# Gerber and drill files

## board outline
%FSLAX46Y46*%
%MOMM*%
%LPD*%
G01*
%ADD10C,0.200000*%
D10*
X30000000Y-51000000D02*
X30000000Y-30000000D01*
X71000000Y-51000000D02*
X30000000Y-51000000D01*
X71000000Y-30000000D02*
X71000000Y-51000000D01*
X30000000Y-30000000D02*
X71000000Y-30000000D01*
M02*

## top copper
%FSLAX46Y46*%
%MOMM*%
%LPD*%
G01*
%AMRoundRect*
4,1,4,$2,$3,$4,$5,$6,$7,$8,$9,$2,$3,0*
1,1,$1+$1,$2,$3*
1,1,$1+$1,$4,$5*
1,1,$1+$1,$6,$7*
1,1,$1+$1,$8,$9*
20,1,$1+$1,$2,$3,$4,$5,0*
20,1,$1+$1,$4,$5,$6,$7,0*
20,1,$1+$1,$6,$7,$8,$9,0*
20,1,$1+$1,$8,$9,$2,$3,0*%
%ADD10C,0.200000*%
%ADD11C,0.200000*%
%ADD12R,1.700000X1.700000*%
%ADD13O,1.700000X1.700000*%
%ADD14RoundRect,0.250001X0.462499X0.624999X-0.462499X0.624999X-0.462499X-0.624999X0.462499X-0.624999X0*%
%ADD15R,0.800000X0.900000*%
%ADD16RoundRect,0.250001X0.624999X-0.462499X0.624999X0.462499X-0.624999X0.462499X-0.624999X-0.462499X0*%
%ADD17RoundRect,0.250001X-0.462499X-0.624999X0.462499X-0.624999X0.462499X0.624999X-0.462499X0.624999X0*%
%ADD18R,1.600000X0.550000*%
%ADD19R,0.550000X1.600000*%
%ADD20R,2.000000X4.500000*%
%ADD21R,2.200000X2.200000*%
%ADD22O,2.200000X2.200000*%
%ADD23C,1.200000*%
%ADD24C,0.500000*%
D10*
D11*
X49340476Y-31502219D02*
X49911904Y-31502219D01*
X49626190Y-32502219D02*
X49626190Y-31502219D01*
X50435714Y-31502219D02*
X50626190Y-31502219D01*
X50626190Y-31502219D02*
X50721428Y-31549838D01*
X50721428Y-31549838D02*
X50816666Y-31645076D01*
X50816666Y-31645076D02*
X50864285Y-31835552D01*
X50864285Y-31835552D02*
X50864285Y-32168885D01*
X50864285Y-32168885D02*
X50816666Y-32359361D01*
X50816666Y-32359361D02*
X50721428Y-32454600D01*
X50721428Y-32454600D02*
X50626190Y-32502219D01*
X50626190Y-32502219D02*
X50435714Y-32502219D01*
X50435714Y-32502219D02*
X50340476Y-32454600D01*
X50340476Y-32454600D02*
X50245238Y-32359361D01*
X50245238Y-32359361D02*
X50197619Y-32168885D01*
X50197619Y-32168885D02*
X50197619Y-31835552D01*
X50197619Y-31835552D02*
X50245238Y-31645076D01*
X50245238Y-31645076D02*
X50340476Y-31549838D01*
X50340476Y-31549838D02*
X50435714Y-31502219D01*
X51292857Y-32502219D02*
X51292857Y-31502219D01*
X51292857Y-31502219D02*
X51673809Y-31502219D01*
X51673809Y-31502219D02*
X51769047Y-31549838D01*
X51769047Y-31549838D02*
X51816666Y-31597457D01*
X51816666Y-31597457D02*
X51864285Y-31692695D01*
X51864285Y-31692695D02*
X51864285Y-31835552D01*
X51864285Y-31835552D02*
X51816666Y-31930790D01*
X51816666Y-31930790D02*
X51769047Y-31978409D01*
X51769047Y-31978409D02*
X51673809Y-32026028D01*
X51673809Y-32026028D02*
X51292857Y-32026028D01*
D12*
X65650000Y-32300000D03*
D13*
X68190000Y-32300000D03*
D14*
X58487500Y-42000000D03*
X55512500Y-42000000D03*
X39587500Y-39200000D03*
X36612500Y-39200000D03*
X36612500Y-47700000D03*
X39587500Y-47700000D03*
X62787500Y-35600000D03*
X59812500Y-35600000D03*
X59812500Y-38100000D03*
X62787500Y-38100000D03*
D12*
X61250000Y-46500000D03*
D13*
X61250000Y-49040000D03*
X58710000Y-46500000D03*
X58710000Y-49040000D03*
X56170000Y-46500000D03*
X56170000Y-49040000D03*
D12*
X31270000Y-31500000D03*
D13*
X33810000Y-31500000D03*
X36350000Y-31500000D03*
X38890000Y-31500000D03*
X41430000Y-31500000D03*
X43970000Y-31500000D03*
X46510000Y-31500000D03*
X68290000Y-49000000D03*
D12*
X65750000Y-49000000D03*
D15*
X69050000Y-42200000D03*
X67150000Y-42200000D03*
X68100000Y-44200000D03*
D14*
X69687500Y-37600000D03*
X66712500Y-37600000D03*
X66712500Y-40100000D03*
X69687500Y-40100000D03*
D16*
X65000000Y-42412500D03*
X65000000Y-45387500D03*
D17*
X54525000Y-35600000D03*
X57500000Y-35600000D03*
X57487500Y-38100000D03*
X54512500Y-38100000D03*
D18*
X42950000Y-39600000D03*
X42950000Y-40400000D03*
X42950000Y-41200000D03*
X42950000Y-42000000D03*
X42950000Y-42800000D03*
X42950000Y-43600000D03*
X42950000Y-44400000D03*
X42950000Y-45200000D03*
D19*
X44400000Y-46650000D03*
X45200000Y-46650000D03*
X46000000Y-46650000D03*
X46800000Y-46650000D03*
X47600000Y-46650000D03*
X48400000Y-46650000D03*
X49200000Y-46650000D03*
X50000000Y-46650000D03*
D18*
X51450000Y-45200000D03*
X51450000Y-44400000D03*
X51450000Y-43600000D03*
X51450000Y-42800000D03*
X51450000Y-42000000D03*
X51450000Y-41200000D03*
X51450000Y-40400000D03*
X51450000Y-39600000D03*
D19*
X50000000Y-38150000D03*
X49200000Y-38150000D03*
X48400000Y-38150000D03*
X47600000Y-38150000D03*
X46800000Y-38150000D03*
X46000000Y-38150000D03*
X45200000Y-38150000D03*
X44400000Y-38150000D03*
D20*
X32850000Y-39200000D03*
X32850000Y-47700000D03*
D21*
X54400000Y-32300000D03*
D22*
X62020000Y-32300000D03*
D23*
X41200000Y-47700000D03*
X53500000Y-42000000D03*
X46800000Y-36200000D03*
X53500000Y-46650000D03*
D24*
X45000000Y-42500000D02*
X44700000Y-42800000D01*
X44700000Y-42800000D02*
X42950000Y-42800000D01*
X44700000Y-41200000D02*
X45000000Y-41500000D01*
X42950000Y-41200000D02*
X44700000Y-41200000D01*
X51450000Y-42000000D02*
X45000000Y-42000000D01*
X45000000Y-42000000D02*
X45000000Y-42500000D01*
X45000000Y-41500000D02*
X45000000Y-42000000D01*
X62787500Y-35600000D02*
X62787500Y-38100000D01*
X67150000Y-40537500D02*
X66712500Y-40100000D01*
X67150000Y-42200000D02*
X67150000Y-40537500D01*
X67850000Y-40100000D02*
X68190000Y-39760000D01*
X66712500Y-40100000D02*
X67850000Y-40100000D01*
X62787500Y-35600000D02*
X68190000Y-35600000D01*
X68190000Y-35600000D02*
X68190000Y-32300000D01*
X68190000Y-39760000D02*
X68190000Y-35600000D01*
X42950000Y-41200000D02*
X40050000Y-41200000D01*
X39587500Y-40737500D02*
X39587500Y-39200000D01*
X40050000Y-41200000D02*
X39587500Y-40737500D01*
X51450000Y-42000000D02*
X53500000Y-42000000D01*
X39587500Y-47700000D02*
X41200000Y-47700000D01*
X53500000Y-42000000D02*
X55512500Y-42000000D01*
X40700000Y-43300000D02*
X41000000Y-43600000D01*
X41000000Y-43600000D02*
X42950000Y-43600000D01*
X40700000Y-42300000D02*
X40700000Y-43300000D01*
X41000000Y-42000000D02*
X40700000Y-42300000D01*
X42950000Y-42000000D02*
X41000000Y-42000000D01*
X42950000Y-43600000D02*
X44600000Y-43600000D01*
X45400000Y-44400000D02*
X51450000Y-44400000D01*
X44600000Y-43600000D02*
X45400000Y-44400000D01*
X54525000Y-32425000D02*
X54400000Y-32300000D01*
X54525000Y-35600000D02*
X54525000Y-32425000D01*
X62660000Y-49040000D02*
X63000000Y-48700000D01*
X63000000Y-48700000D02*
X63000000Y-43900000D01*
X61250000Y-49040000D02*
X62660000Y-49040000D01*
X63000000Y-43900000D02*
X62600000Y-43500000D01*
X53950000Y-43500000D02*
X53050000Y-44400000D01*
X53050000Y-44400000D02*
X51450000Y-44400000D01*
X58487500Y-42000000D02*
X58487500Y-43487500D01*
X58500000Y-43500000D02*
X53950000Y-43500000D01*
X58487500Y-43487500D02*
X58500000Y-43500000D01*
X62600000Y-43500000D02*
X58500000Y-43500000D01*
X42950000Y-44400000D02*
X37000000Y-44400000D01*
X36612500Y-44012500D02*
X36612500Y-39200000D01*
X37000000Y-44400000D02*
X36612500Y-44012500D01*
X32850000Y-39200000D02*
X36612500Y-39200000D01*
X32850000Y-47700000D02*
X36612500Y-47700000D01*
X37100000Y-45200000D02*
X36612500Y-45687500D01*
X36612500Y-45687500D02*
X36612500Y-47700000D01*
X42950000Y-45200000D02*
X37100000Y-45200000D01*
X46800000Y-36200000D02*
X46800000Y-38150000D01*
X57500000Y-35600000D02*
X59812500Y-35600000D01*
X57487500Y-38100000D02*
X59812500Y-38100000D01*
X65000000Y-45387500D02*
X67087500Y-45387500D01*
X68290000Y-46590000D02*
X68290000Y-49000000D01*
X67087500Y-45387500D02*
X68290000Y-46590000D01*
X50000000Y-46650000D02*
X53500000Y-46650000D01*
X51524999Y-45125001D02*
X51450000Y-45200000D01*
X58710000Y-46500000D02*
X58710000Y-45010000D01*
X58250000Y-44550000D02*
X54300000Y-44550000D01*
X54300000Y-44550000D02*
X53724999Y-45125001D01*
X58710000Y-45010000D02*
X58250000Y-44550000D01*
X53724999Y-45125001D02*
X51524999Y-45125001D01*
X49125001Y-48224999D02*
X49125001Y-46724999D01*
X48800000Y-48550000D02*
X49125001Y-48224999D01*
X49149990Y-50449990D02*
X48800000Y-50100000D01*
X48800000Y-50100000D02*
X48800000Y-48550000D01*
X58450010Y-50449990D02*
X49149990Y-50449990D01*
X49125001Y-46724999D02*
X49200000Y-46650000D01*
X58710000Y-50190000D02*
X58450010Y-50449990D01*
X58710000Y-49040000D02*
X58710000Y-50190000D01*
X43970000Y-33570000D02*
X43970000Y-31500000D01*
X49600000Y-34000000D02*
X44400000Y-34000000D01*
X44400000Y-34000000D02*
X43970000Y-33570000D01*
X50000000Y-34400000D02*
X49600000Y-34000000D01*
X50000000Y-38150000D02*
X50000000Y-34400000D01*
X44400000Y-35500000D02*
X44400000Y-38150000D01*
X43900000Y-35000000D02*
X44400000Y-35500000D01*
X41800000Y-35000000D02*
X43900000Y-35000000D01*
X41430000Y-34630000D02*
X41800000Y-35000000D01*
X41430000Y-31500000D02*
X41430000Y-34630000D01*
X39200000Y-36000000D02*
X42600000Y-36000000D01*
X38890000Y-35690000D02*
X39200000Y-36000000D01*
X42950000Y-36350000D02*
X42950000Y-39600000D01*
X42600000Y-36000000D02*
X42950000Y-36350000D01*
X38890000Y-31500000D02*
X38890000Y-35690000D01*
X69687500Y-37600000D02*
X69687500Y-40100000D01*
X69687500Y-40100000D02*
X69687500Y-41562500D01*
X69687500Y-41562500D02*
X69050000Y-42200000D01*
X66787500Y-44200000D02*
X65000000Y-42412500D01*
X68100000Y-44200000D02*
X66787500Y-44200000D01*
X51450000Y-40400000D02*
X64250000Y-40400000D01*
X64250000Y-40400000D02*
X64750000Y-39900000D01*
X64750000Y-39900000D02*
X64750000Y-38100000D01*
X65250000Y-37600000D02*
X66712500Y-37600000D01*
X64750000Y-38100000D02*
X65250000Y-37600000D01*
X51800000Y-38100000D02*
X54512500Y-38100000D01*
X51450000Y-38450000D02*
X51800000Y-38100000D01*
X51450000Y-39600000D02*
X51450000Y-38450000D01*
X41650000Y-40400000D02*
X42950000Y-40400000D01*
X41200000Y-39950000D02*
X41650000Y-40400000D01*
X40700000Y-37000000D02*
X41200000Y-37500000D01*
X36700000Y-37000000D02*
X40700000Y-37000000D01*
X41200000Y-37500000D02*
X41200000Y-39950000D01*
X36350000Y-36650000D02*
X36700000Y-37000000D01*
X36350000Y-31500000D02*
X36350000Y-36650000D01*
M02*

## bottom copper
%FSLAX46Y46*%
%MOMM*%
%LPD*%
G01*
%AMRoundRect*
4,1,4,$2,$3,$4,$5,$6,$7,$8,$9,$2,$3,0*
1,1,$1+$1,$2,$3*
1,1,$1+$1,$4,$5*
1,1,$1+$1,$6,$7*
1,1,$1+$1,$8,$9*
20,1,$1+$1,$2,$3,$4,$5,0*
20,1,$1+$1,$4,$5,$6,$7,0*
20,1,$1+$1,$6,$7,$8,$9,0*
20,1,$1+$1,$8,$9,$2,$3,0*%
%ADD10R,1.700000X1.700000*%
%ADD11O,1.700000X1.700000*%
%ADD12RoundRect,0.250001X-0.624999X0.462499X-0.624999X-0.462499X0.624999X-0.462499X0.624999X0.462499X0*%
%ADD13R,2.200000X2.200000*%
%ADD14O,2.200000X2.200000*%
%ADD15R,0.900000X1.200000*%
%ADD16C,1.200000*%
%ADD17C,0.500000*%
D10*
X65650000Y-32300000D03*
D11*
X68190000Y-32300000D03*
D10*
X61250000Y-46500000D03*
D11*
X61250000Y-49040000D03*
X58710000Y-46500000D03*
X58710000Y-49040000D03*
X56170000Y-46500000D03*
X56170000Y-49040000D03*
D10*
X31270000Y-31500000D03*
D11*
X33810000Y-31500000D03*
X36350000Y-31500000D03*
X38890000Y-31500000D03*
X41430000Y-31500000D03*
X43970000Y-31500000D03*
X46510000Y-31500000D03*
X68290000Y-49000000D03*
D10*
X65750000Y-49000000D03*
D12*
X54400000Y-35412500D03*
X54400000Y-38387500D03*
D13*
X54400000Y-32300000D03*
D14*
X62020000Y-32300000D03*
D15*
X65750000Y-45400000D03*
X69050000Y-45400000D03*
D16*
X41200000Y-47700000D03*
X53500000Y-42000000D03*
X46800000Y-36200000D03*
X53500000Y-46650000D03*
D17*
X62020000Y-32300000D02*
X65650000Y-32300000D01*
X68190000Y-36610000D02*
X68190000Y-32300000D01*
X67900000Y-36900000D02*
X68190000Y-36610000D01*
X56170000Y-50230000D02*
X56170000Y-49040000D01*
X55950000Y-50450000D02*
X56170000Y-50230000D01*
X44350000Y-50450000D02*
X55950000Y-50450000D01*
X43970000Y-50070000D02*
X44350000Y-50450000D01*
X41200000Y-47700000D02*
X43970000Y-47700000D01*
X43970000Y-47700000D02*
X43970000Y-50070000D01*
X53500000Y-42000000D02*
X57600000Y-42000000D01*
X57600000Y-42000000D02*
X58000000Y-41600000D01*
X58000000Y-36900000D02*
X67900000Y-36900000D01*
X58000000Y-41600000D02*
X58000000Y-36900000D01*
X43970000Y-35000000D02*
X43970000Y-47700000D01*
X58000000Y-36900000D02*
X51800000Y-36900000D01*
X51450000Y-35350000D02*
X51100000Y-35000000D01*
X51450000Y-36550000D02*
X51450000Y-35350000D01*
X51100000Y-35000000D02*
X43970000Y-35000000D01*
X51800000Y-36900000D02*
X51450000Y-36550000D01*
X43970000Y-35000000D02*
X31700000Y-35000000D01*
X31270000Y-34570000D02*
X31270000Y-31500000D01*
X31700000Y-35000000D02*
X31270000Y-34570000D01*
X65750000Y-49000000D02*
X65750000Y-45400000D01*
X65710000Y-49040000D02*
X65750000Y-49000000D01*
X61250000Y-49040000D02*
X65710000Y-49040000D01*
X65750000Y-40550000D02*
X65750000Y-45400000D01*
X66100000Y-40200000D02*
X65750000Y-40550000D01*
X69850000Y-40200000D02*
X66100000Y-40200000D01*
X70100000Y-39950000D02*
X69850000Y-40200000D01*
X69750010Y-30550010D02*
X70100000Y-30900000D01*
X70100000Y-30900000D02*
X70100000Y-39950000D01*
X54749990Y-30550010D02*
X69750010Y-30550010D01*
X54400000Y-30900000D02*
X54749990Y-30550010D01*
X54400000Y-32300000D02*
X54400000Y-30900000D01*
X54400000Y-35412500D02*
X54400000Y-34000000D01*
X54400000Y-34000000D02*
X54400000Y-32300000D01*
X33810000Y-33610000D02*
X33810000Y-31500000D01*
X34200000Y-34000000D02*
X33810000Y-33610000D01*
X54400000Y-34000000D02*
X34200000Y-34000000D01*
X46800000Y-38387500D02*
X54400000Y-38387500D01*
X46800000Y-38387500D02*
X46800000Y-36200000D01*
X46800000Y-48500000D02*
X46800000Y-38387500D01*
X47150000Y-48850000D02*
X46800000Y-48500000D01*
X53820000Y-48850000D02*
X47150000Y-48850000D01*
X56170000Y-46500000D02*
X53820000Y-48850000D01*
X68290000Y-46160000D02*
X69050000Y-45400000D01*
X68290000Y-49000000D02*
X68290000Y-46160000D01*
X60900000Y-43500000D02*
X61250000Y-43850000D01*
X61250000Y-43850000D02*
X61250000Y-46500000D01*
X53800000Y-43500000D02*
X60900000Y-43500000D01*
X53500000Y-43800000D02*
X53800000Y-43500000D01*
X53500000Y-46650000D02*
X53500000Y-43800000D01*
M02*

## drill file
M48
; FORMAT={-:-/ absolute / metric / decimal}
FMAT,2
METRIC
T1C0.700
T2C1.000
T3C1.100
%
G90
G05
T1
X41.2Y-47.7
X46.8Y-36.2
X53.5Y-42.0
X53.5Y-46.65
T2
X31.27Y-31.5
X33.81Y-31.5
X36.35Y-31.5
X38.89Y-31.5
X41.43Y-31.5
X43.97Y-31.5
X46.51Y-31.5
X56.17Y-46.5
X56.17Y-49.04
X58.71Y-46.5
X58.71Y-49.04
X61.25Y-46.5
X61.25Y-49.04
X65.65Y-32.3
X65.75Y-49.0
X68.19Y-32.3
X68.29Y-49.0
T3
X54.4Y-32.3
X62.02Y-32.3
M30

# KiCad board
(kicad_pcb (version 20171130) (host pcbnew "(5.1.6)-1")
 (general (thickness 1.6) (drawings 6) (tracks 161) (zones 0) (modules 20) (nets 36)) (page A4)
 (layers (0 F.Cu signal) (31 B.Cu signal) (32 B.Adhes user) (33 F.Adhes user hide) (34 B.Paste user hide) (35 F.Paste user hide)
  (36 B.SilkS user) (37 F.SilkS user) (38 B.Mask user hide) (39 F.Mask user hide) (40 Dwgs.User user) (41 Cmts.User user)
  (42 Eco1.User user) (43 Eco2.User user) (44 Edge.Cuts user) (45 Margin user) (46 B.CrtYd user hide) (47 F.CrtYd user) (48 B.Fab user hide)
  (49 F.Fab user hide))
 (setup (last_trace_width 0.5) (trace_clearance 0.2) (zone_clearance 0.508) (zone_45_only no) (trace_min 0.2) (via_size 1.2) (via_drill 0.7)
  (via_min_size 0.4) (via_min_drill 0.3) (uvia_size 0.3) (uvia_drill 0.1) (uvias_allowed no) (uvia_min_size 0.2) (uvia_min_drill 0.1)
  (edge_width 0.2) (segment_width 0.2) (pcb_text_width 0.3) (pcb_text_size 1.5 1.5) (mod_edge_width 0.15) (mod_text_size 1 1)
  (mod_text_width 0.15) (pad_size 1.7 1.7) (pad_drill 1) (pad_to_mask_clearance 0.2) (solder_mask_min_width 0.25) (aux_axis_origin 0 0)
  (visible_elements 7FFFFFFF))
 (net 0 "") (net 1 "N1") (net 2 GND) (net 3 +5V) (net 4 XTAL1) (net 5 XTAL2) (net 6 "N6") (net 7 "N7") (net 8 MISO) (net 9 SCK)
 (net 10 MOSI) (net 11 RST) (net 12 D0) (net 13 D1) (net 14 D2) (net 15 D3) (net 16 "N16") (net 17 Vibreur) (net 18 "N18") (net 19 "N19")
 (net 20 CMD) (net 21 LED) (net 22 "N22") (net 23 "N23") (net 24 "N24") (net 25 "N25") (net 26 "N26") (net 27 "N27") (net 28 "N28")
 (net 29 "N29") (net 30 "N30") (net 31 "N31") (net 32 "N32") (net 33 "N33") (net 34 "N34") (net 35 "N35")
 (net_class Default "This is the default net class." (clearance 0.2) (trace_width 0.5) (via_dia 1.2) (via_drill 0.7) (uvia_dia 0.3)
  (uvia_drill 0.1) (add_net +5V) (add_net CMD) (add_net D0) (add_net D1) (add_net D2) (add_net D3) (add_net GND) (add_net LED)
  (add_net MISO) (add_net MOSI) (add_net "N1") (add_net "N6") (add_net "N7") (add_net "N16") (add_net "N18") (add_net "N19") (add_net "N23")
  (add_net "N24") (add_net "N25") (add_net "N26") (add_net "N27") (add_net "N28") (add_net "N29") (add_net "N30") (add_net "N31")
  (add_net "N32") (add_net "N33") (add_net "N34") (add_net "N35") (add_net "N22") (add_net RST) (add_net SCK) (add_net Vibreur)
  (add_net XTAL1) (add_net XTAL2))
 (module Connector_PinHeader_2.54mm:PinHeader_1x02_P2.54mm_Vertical (layer F.Cu) (at 65.65 32.3 90)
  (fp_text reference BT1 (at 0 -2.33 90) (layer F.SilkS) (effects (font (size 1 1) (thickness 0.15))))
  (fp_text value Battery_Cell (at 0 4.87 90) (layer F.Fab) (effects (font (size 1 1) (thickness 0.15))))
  (pad 1 thru_hole rect (at 0 0 90) (size 1.7 1.7) (drill 1) (layers *.Cu *.Mask) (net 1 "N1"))
  (pad 2 thru_hole oval (at 0 2.54 90) (size 1.7 1.7) (drill 1) (layers *.Cu *.Mask) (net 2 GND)))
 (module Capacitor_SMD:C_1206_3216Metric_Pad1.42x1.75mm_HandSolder (layer F.Cu) (at 57 42 180)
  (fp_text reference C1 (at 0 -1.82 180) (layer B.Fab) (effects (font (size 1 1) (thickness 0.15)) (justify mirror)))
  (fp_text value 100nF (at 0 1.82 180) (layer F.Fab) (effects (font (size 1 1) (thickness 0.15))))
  (pad 1 smd roundrect (at -1.4875 0 180) (size 1.425 1.75) (layers F.Cu F.Paste F.Mask) (roundrect_rratio 0.175439) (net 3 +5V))
  (pad 2 smd roundrect (at 1.4875 0 180) (size 1.425 1.75) (layers F.Cu F.Paste F.Mask) (roundrect_rratio 0.175439) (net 2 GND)))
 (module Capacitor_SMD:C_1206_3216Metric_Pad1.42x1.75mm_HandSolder (layer F.Cu) (at 38.1 39.2 180)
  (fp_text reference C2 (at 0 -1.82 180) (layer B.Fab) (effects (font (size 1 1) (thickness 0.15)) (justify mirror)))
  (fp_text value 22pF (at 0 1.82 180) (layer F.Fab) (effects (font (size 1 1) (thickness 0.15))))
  (pad 1 smd roundrect (at -1.4875 0 180) (size 1.425 1.75) (layers F.Cu F.Paste F.Mask) (roundrect_rratio 0.175439) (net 2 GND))
  (pad 2 smd roundrect (at 1.4875 0 180) (size 1.425 1.75) (layers F.Cu F.Paste F.Mask) (roundrect_rratio 0.175439) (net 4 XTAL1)))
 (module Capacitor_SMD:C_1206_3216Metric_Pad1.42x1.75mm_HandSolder (layer F.Cu) (at 38.1 47.7 180)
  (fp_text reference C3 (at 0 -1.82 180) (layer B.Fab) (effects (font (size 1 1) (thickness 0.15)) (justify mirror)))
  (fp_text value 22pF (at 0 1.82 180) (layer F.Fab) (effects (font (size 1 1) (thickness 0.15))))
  (pad 2 smd roundrect (at 1.4875 0 180) (size 1.425 1.75) (layers F.Cu F.Paste F.Mask) (roundrect_rratio 0.175439) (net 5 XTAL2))
  (pad 1 smd roundrect (at -1.4875 0 180) (size 1.425 1.75) (layers F.Cu F.Paste F.Mask) (roundrect_rratio 0.175439) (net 2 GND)))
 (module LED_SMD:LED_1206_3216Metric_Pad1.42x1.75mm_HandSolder (layer F.Cu) (at 61.3 35.6 180)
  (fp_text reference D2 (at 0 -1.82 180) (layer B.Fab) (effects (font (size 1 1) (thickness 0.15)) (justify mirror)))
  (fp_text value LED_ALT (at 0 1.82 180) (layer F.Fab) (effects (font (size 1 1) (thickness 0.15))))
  (pad 1 smd roundrect (at -1.4875 0 180) (size 1.425 1.75) (layers F.Cu F.Paste F.Mask) (roundrect_rratio 0.175439) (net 2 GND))
  (pad 2 smd roundrect (at 1.4875 0 180) (size 1.425 1.75) (layers F.Cu F.Paste F.Mask) (roundrect_rratio 0.175439) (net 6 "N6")))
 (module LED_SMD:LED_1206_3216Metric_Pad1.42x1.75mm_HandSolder (layer F.Cu) (at 61.3 38.1 180)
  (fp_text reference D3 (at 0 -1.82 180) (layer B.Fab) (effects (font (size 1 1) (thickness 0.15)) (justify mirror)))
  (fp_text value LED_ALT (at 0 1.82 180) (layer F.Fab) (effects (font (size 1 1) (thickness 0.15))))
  (pad 2 smd roundrect (at 1.4875 0 180) (size 1.425 1.75) (layers F.Cu F.Paste F.Mask) (roundrect_rratio 0.175439) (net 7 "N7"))
  (pad 1 smd roundrect (at -1.4875 0 180) (size 1.425 1.75) (layers F.Cu F.Paste F.Mask) (roundrect_rratio 0.175439) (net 2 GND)))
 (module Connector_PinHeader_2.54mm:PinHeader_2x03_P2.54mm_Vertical (layer F.Cu) (at 61.25 46.5 270)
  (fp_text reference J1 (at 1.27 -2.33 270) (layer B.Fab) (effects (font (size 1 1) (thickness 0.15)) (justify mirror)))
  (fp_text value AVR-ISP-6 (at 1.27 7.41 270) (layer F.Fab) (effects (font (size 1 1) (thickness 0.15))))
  (pad 1 thru_hole rect (at 0 0 270) (size 1.7 1.7) (drill 1) (layers *.Cu *.Mask) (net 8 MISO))
  (pad 2 thru_hole oval (at 2.54 0 270) (size 1.7 1.7) (drill 1) (layers *.Cu *.Mask) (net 3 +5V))
  (pad 3 thru_hole oval (at 0 2.54 270) (size 1.7 1.7) (drill 1) (layers *.Cu *.Mask) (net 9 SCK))
  (pad 4 thru_hole oval (at 2.54 2.54 270) (size 1.7 1.7) (drill 1) (layers *.Cu *.Mask) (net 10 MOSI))
  (pad 5 thru_hole oval (at 0 5.08 270) (size 1.7 1.7) (drill 1) (layers *.Cu *.Mask) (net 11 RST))
  (pad 6 thru_hole oval (at 2.54 5.08 270) (size 1.7 1.7) (drill 1) (layers *.Cu *.Mask) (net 2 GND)))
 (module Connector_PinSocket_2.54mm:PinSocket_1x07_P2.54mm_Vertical (layer F.Cu) (at 31.27 31.5 90)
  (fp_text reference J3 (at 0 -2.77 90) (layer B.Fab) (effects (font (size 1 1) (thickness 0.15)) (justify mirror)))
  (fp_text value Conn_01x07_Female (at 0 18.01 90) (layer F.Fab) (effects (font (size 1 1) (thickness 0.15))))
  (pad 1 thru_hole rect (at 0 0 90) (size 1.7 1.7) (drill 1) (layers *.Cu *.Mask) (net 2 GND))
  (pad 2 thru_hole oval (at 0 2.54 90) (size 1.7 1.7) (drill 1) (layers *.Cu *.Mask) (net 3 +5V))
  (pad 3 thru_hole oval (at 0 5.08 90) (size 1.7 1.7) (drill 1) (layers *.Cu *.Mask) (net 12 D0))
  (pad 4 thru_hole oval (at 0 7.62 90) (size 1.7 1.7) (drill 1) (layers *.Cu *.Mask) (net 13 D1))
  (pad 5 thru_hole oval (at 0 10.16 90) (size 1.7 1.7) (drill 1) (layers *.Cu *.Mask) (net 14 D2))
  (pad 6 thru_hole oval (at 0 12.7 90) (size 1.7 1.7) (drill 1) (layers *.Cu *.Mask) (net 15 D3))
  (pad 7 thru_hole oval (at 0 15.24 90) (size 1.7 1.7) (drill 1) (layers *.Cu *.Mask) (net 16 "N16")))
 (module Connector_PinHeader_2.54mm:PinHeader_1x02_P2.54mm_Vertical (layer F.Cu) (at 65.75 49 90)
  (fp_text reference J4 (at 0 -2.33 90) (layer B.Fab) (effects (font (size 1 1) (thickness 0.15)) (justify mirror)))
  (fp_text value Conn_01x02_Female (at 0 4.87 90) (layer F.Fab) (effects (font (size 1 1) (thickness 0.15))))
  (pad 2 thru_hole oval (at 0 2.54 90) (size 1.7 1.7) (drill 1) (layers *.Cu *.Mask) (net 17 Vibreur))
  (pad 1 thru_hole rect (at 0 0 90) (size 1.7 1.7) (drill 1) (layers *.Cu *.Mask) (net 3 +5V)))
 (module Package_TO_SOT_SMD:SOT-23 (layer F.Cu) (at 68.1 43.2 270)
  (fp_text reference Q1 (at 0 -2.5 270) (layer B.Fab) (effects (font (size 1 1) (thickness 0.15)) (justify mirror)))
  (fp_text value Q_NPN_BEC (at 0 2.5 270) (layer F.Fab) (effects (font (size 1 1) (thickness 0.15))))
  (pad 1 smd rect (at -1 -0.95 270) (size 0.9 0.8) (layers F.Cu F.Paste F.Mask) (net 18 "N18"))
  (pad 2 smd rect (at -1 0.95 270) (size 0.9 0.8) (layers F.Cu F.Paste F.Mask) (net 2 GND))
  (pad 3 smd rect (at 1 0 270) (size 0.9 0.8) (layers F.Cu F.Paste F.Mask) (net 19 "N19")))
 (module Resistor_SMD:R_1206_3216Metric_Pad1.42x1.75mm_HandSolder (layer B.Cu) (at 54.4 36.9 270)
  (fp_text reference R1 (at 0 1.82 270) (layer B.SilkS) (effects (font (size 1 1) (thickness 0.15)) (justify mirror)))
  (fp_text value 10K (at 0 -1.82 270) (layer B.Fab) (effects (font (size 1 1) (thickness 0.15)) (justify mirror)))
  (pad 1 smd roundrect (at -1.4875 0 270) (size 1.425 1.75) (layers B.Cu B.Paste B.Mask) (roundrect_rratio 0.175439) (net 3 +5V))
  (pad 2 smd roundrect (at 1.4875 0 270) (size 1.425 1.75) (layers B.Cu B.Paste B.Mask) (roundrect_rratio 0.175439) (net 11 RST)))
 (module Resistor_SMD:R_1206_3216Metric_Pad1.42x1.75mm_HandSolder (layer F.Cu) (at 68.2 37.6 180)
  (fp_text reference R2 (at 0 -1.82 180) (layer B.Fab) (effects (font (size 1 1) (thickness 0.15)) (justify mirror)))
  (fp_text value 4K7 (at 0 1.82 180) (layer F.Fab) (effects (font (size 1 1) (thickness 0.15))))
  (pad 1 smd roundrect (at -1.4875 0 180) (size 1.425 1.75) (layers F.Cu F.Paste F.Mask) (roundrect_rratio 0.175439) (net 18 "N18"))
  (pad 2 smd roundrect (at 1.4875 0 180) (size 1.425 1.75) (layers F.Cu F.Paste F.Mask) (roundrect_rratio 0.175439) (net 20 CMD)))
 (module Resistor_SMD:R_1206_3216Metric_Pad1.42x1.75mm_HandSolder (layer F.Cu) (at 68.2 40.1 180)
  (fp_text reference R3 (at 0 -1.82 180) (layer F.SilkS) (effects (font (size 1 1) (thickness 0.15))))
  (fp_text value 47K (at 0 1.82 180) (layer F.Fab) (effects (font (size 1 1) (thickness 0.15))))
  (pad 2 smd roundrect (at 1.4875 0 180) (size 1.425 1.75) (layers F.Cu F.Paste F.Mask) (roundrect_rratio 0.175439) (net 2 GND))
  (pad 1 smd roundrect (at -1.4875 0 180) (size 1.425 1.75) (layers F.Cu F.Paste F.Mask) (roundrect_rratio 0.175439) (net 18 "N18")))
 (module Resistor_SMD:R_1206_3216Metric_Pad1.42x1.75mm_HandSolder (layer F.Cu) (at 65 43.9 90)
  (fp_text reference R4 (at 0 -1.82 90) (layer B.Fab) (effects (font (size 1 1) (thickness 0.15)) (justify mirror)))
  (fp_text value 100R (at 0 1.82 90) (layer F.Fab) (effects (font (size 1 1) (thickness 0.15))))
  (pad 2 smd roundrect (at 1.4875 0 90) (size 1.425 1.75) (layers F.Cu F.Paste F.Mask) (roundrect_rratio 0.175439) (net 19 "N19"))
  (pad 1 smd roundrect (at -1.4875 0 90) (size 1.425 1.75) (layers F.Cu F.Paste F.Mask) (roundrect_rratio 0.175439) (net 17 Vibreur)))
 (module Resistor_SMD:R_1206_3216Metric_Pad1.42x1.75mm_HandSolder (layer F.Cu) (at 56.0125 35.6)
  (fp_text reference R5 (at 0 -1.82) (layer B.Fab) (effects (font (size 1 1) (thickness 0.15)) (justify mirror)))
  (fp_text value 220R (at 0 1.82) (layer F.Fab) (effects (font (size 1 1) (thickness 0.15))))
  (pad 1 smd roundrect (at -1.4875 0) (size 1.425 1.75) (layers F.Cu F.Paste F.Mask) (roundrect_rratio 0.175439) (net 3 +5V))
  (pad 2 smd roundrect (at 1.4875 0) (size 1.425 1.75) (layers F.Cu F.Paste F.Mask) (roundrect_rratio 0.175439) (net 6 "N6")))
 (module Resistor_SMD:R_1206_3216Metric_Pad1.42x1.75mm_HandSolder (layer F.Cu) (at 56 38.1)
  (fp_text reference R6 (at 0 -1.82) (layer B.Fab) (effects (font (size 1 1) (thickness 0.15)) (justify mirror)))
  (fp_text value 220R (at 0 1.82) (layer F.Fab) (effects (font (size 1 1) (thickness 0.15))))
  (pad 2 smd roundrect (at 1.4875 0) (size 1.425 1.75) (layers F.Cu F.Paste F.Mask) (roundrect_rratio 0.175439) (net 7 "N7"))
  (pad 1 smd roundrect (at -1.4875 0) (size 1.425 1.75) (layers F.Cu F.Paste F.Mask) (roundrect_rratio 0.175439) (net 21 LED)))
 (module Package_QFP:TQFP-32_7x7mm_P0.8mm (layer F.Cu) (at 47.2 42.4)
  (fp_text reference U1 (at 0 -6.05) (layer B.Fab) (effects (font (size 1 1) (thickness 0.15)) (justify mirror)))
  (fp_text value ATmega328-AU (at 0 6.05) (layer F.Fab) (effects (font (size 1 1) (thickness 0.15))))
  (pad 1 smd rect (at -4.25 -2.8) (size 1.6 0.55) (layers F.Cu F.Paste F.Mask) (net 13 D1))
  (pad 2 smd rect (at -4.25 -2) (size 1.6 0.55) (layers F.Cu F.Paste F.Mask) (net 12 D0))
  (pad 3 smd rect (at -4.25 -1.2) (size 1.6 0.55) (layers F.Cu F.Paste F.Mask) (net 2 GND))
  (pad 4 smd rect (at -4.25 -0.4) (size 1.6 0.55) (layers F.Cu F.Paste F.Mask) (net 3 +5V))
  (pad 5 smd rect (at -4.25 0.4) (size 1.6 0.55) (layers F.Cu F.Paste F.Mask) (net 2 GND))
  (pad 6 smd rect (at -4.25 1.2) (size 1.6 0.55) (layers F.Cu F.Paste F.Mask) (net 3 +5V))
  (pad 7 smd rect (at -4.25 2) (size 1.6 0.55) (layers F.Cu F.Paste F.Mask) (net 4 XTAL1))
  (pad 8 smd rect (at -4.25 2.8) (size 1.6 0.55) (layers F.Cu F.Paste F.Mask) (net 5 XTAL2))
  (pad 9 smd rect (at -2.8 4.25 90) (size 1.6 0.55) (layers F.Cu F.Paste F.Mask) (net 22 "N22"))
  (pad 10 smd rect (at -2 4.25 90) (size 1.6 0.55) (layers F.Cu F.Paste F.Mask) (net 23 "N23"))
  (pad 11 smd rect (at -1.2 4.25 90) (size 1.6 0.55) (layers F.Cu F.Paste F.Mask) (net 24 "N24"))
  (pad 12 smd rect (at -0.4 4.25 90) (size 1.6 0.55) (layers F.Cu F.Paste F.Mask) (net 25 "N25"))
  (pad 13 smd rect (at 0.4 4.25 90) (size 1.6 0.55) (layers F.Cu F.Paste F.Mask) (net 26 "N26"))
  (pad 14 smd rect (at 1.2 4.25 90) (size 1.6 0.55) (layers F.Cu F.Paste F.Mask) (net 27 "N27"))
  (pad 15 smd rect (at 2 4.25 90) (size 1.6 0.55) (layers F.Cu F.Paste F.Mask) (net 10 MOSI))
  (pad 16 smd rect (at 2.8 4.25 90) (size 1.6 0.55) (layers F.Cu F.Paste F.Mask) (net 8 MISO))
  (pad 17 smd rect (at 4.25 2.8) (size 1.6 0.55) (layers F.Cu F.Paste F.Mask) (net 9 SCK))
  (pad 18 smd rect (at 4.25 2) (size 1.6 0.55) (layers F.Cu F.Paste F.Mask) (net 3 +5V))
  (pad 19 smd rect (at 4.25 1.2) (size 1.6 0.55) (layers F.Cu F.Paste F.Mask) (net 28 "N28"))
  (pad 20 smd rect (at 4.25 0.4) (size 1.6 0.55) (layers F.Cu F.Paste F.Mask) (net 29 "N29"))
  (pad 21 smd rect (at 4.25 -0.4) (size 1.6 0.55) (layers F.Cu F.Paste F.Mask) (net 2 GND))
  (pad 22 smd rect (at 4.25 -1.2) (size 1.6 0.55) (layers F.Cu F.Paste F.Mask) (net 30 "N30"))
  (pad 23 smd rect (at 4.25 -2) (size 1.6 0.55) (layers F.Cu F.Paste F.Mask) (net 20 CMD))
  (pad 24 smd rect (at 4.25 -2.8) (size 1.6 0.55) (layers F.Cu F.Paste F.Mask) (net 21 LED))
  (pad 25 smd rect (at 2.8 -4.25 90) (size 1.6 0.55) (layers F.Cu F.Paste F.Mask) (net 15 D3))
  (pad 26 smd rect (at 2 -4.25 90) (size 1.6 0.55) (layers F.Cu F.Paste F.Mask) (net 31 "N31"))
  (pad 27 smd rect (at 1.2 -4.25 90) (size 1.6 0.55) (layers F.Cu F.Paste F.Mask) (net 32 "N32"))
  (pad 28 smd rect (at 0.4 -4.25 90) (size 1.6 0.55) (layers F.Cu F.Paste F.Mask) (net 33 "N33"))
  (pad 29 smd rect (at -0.4 -4.25 90) (size 1.6 0.55) (layers F.Cu F.Paste F.Mask) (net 11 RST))
  (pad 30 smd rect (at -1.2 -4.25 90) (size 1.6 0.55) (layers F.Cu F.Paste F.Mask) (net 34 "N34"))
  (pad 31 smd rect (at -2 -4.25 90) (size 1.6 0.55) (layers F.Cu F.Paste F.Mask) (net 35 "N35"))
  (pad 32 smd rect (at -2.8 -4.25 90) (size 1.6 0.55) (layers F.Cu F.Paste F.Mask) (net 14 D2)))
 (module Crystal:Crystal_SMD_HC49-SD (layer F.Cu) (at 32.85 43.45 270)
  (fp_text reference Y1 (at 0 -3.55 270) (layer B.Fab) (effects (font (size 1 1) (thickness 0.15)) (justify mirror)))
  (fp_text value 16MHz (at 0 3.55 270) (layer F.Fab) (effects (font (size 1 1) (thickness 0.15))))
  (pad 1 smd rect (at -4.25 0 270) (size 4.5 2) (layers F.Cu F.Paste F.Mask) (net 4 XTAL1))
  (pad 2 smd rect (at 4.25 0 270) (size 4.5 2) (layers F.Cu F.Paste F.Mask) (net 5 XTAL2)))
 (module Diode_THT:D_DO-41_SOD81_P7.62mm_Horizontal (layer F.Cu) (at 54.4 32.3)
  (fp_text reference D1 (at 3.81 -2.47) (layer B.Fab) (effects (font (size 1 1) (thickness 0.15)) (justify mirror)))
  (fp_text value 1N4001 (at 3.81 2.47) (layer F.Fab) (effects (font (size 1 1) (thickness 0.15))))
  (pad 1 thru_hole rect (at 0 0) (size 2.2 2.2) (drill 1.1) (layers *.Cu *.Mask) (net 3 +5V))
  (pad 2 thru_hole oval (at 7.62 0) (size 2.2 2.2) (drill 1.1) (layers *.Cu *.Mask) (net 1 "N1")))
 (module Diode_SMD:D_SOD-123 (layer B.Cu) (at 67.4 45.4)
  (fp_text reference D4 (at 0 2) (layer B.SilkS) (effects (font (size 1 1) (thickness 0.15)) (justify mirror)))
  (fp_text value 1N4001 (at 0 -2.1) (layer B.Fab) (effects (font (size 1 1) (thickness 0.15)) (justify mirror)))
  (pad 1 smd rect (at -1.65 0) (size 0.9 1.2) (layers B.Cu B.Paste B.Mask) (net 3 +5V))
  (pad 2 smd rect (at 1.65 0) (size 0.9 1.2) (layers B.Cu B.Paste B.Mask) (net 17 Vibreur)))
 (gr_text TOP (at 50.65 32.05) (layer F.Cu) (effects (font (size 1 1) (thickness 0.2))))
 (gr_line (start 30 51) (end 30 30) (layer Edge.Cuts) (width 0.2))
 (gr_line (start 71 51) (end 30 51) (layer Edge.Cuts) (width 0.2))
 (gr_line (start 71 30) (end 71 51) (layer Edge.Cuts) (width 0.2))
 (gr_line (start 30 30) (end 71 30) (layer Edge.Cuts) (width 0.2))
 (segment (start 62.02 32.3) (end 65.65 32.3) (width 0.5) (layer B.Cu) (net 1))
 (segment (start 45 42.5) (end 44.7 42.8) (width 0.5) (layer F.Cu) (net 2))
 (segment (start 44.7 42.8) (end 42.95 42.8) (width 0.5) (layer F.Cu) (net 2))
 (segment (start 44.7 41.2) (end 45 41.5) (width 0.5) (layer F.Cu) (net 2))
 (segment (start 42.95 41.2) (end 44.7 41.2) (width 0.5) (layer F.Cu) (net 2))
 (segment (start 51.45 42) (end 45 42) (width 0.5) (layer F.Cu) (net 2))
 (segment (start 45 42) (end 45 42.5) (width 0.5) (layer F.Cu) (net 2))
 (segment (start 45 41.5) (end 45 42) (width 0.5) (layer F.Cu) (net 2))
 (segment (start 62.7875 35.6) (end 62.7875 38.1) (width 0.5) (layer F.Cu) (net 2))
 (segment (start 67.15 40.5375) (end 66.7125 40.1) (width 0.5) (layer F.Cu) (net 2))
 (segment (start 67.15 42.2) (end 67.15 40.5375) (width 0.5) (layer F.Cu) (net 2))
 (segment (start 67.85 40.1) (end 68.19 39.76) (width 0.5) (layer F.Cu) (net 2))
 (segment (start 66.7125 40.1) (end 67.85 40.1) (width 0.5) (layer F.Cu) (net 2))
 (segment (start 62.7875 35.6) (end 68.19 35.6) (width 0.5) (layer F.Cu) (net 2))
 (segment (start 68.19 35.6) (end 68.19 32.3) (width 0.5) (layer F.Cu) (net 2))
 (segment (start 68.19 39.76) (end 68.19 35.6) (width 0.5) (layer F.Cu) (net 2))
 (segment (start 42.95 41.2) (end 40.05 41.2) (width 0.5) (layer F.Cu) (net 2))
 (segment (start 39.5875 40.7375) (end 39.5875 39.2) (width 0.5) (layer F.Cu) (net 2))
 (segment (start 40.05 41.2) (end 39.5875 40.7375) (width 0.5) (layer F.Cu) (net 2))
 (segment (start 68.19 36.61) (end 68.19 32.3) (width 0.5) (layer B.Cu) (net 2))
 (segment (start 67.9 36.9) (end 68.19 36.61) (width 0.5) (layer B.Cu) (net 2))
 (segment (start 56.17 50.23) (end 56.17 49.04) (width 0.5) (layer B.Cu) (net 2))
 (segment (start 55.95 50.45) (end 56.17 50.23) (width 0.5) (layer B.Cu) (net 2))
 (segment (start 44.35 50.45) (end 55.95 50.45) (width 0.5) (layer B.Cu) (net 2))
 (segment (start 43.97 50.07) (end 44.35 50.45) (width 0.5) (layer B.Cu) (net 2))
 (segment (start 51.45 42) (end 53.5 42) (width 0.5) (layer F.Cu) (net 2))
 (via (at 41.2 47.7) (size 1.2) (drill 0.7) (layers F.Cu B.Cu) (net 2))
 (segment (start 39.5875 47.7) (end 41.2 47.7) (width 0.5) (layer F.Cu) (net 2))
 (segment (start 41.2 47.7) (end 43.97 47.7) (width 0.5) (layer B.Cu) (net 2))
 (segment (start 43.97 47.7) (end 43.97 50.07) (width 0.5) (layer B.Cu) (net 2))
 (segment (start 53.5 42) (end 55.5125 42) (width 0.5) (layer F.Cu) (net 2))
 (via (at 53.5 42) (size 1.2) (drill 0.7) (layers F.Cu B.Cu) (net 2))
 (segment (start 53.5 42) (end 57.6 42) (width 0.5) (layer B.Cu) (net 2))
 (segment (start 57.6 42) (end 58 41.6) (width 0.5) (layer B.Cu) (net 2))
 (segment (start 58 36.9) (end 67.9 36.9) (width 0.5) (layer B.Cu) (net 2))
 (segment (start 58 41.6) (end 58 36.9) (width 0.5) (layer B.Cu) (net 2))
 (segment (start 43.97 35) (end 43.97 47.7) (width 0.5) (layer B.Cu) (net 2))
 (segment (start 58 36.9) (end 51.8 36.9) (width 0.5) (layer B.Cu) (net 2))
 (segment (start 51.45 35.35) (end 51.1 35) (width 0.5) (layer B.Cu) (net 2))
 (segment (start 51.45 36.55) (end 51.45 35.35) (width 0.5) (layer B.Cu) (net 2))
 (segment (start 51.1 35) (end 43.97 35) (width 0.5) (layer B.Cu) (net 2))
 (segment (start 51.8 36.9) (end 51.45 36.55) (width 0.5) (layer B.Cu) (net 2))
 (segment (start 43.97 35) (end 31.7 35) (width 0.5) (layer B.Cu) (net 2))
 (segment (start 31.27 34.57) (end 31.27 31.5) (width 0.5) (layer B.Cu) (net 2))
 (segment (start 31.7 35) (end 31.27 34.57) (width 0.5) (layer B.Cu) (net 2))
 (segment (start 40.7 43.3) (end 41 43.6) (width 0.5) (layer F.Cu) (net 3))
 (segment (start 41 43.6) (end 42.95 43.6) (width 0.5) (layer F.Cu) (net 3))
 (segment (start 40.7 42.3) (end 40.7 43.3) (width 0.5) (layer F.Cu) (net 3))
 (segment (start 41 42) (end 40.7 42.3) (width 0.5) (layer F.Cu) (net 3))
 (segment (start 42.95 42) (end 41 42) (width 0.5) (layer F.Cu) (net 3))
 (segment (start 42.95 43.6) (end 44.6 43.6) (width 0.5) (layer F.Cu) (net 3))
 (segment (start 45.4 44.4) (end 51.45 44.4) (width 0.5) (layer F.Cu) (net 3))
 (segment (start 44.6 43.6) (end 45.4 44.4) (width 0.5) (layer F.Cu) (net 3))
 (segment (start 65.75 49) (end 65.75 45.4) (width 0.5) (layer B.Cu) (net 3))
 (segment (start 65.71 49.04) (end 65.75 49) (width 0.5) (layer B.Cu) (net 3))
 (segment (start 61.25 49.04) (end 65.71 49.04) (width 0.5) (layer B.Cu) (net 3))
 (segment (start 54.525 32.425) (end 54.4 32.3) (width 0.5) (layer F.Cu) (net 3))
 (segment (start 54.525 35.6) (end 54.525 32.425) (width 0.5) (layer F.Cu) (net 3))
 (segment (start 62.66 49.04) (end 63 48.7) (width 0.5) (layer F.Cu) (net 3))
 (segment (start 63 48.7) (end 63 43.9) (width 0.5) (layer F.Cu) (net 3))
 (segment (start 61.25 49.04) (end 62.66 49.04) (width 0.5) (layer F.Cu) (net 3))
 (segment (start 63 43.9) (end 62.6 43.5) (width 0.5) (layer F.Cu) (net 3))
 (segment (start 53.95 43.5) (end 53.05 44.4) (width 0.5) (layer F.Cu) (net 3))
 (segment (start 53.05 44.4) (end 51.45 44.4) (width 0.5) (layer F.Cu) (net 3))
 (segment (start 58.4875 42) (end 58.4875 43.4875) (width 0.5) (layer F.Cu) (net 3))
 (segment (start 58.5 43.5) (end 53.95 43.5) (width 0.5) (layer F.Cu) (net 3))
 (segment (start 58.4875 43.4875) (end 58.5 43.5) (width 0.5) (layer F.Cu) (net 3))
 (segment (start 62.6 43.5) (end 58.5 43.5) (width 0.5) (layer F.Cu) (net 3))
 (segment (start 65.75 40.55) (end 65.75 45.4) (width 0.5) (layer B.Cu) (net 3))
 (segment (start 66.1 40.2) (end 65.75 40.55) (width 0.5) (layer B.Cu) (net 3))
 (segment (start 69.85 40.2) (end 66.1 40.2) (width 0.5) (layer B.Cu) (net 3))
 (segment (start 70.1 39.95) (end 69.85 40.2) (width 0.5) (layer B.Cu) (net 3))
 (segment (start 69.75001 30.55001) (end 70.1 30.9) (width 0.5) (layer B.Cu) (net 3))
 (segment (start 70.1 30.9) (end 70.1 39.95) (width 0.5) (layer B.Cu) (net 3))
 (segment (start 54.74999 30.55001) (end 69.75001 30.55001) (width 0.5) (layer B.Cu) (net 3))
 (segment (start 54.4 30.9) (end 54.74999 30.55001) (width 0.5) (layer B.Cu) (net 3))
 (segment (start 54.4 32.3) (end 54.4 30.9) (width 0.5) (layer B.Cu) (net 3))
 (segment (start 54.4 35.4125) (end 54.4 34) (width 0.5) (layer B.Cu) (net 3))
 (segment (start 54.4 34) (end 54.4 32.3) (width 0.5) (layer B.Cu) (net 3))
 (segment (start 33.81 33.61) (end 33.81 31.5) (width 0.5) (layer B.Cu) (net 3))
 (segment (start 34.2 34) (end 33.81 33.61) (width 0.5) (layer B.Cu) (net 3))
 (segment (start 54.4 34) (end 34.2 34) (width 0.5) (layer B.Cu) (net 3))
 (segment (start 42.95 44.4) (end 37 44.4) (width 0.5) (layer F.Cu) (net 4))
 (segment (start 36.6125 44.0125) (end 36.6125 39.2) (width 0.5) (layer F.Cu) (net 4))
 (segment (start 37 44.4) (end 36.6125 44.0125) (width 0.5) (layer F.Cu) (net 4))
 (segment (start 32.85 39.2) (end 36.6125 39.2) (width 0.5) (layer F.Cu) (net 4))
 (segment (start 32.85 47.7) (end 36.6125 47.7) (width 0.5) (layer F.Cu) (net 5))
 (segment (start 37.1 45.2) (end 36.6125 45.6875) (width 0.5) (layer F.Cu) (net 5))
 (segment (start 36.6125 45.6875) (end 36.6125 47.7) (width 0.5) (layer F.Cu) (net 5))
 (segment (start 42.95 45.2) (end 37.1 45.2) (width 0.5) (layer F.Cu) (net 5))
 (segment (start 46.8 38.3875) (end 54.4 38.3875) (width 0.5) (layer B.Cu) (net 11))
 (via (at 46.8 36.2) (size 1.2) (drill 0.7) (layers F.Cu B.Cu) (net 11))
 (segment (start 46.8 38.3875) (end 46.8 36.2) (width 0.5) (layer B.Cu) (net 11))
 (segment (start 46.8 36.2) (end 46.8 38.15) (width 0.5) (layer F.Cu) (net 11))
 (segment (start 46.8 48.5) (end 46.8 38.3875) (width 0.5) (layer B.Cu) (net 11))
 (segment (start 47.15 48.85) (end 46.8 48.5) (width 0.5) (layer B.Cu) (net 11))
 (segment (start 53.82 48.85) (end 47.15 48.85) (width 0.5) (layer B.Cu) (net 11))
 (segment (start 56.17 46.5) (end 53.82 48.85) (width 0.5) (layer B.Cu) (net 11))
 (segment (start 57.5 35.6) (end 59.8125 35.6) (width 0.5) (layer F.Cu) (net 6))
 (segment (start 57.4875 38.1) (end 59.8125 38.1) (width 0.5) (layer F.Cu) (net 7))
 (segment (start 65 45.3875) (end 67.0875 45.3875) (width 0.5) (layer F.Cu) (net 17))
 (segment (start 68.29 46.59) (end 68.29 49) (width 0.5) (layer F.Cu) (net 17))
 (segment (start 67.0875 45.3875) (end 68.29 46.59) (width 0.5) (layer F.Cu) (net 17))
 (segment (start 68.29 46.16) (end 69.05 45.4) (width 0.5) (layer B.Cu) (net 17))
 (segment (start 68.29 49) (end 68.29 46.16) (width 0.5) (layer B.Cu) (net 17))
 (via (at 53.5 46.65) (size 1.2) (drill 0.7) (layers F.Cu B.Cu) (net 8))
 (segment (start 50 46.65) (end 53.5 46.65) (width 0.5) (layer F.Cu) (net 8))
 (segment (start 60.9 43.5) (end 61.25 43.85) (width 0.5) (layer B.Cu) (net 8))
 (segment (start 61.25 43.85) (end 61.25 46.5) (width 0.5) (layer B.Cu) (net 8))
 (segment (start 53.8 43.5) (end 60.9 43.5) (width 0.5) (layer B.Cu) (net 8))
 (segment (start 53.5 43.8) (end 53.8 43.5) (width 0.5) (layer B.Cu) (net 8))
 (segment (start 53.5 46.65) (end 53.5 43.8) (width 0.5) (layer B.Cu) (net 8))
 (segment (start 51.524999 45.125001) (end 51.45 45.2) (width 0.5) (layer F.Cu) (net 9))
 (segment (start 58.71 46.5) (end 58.71 45.01) (width 0.5) (layer F.Cu) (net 9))
 (segment (start 58.25 44.55) (end 54.3 44.55) (width 0.5) (layer F.Cu) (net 9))
 (segment (start 54.3 44.55) (end 53.724999 45.125001) (width 0.5) (layer F.Cu) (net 9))
 (segment (start 58.71 45.01) (end 58.25 44.55) (width 0.5) (layer F.Cu) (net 9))
 (segment (start 53.724999 45.125001) (end 51.524999 45.125001) (width 0.5) (layer F.Cu) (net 9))
 (segment (start 49.125001 48.224999) (end 49.125001 46.724999) (width 0.5) (layer F.Cu) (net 10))
 (segment (start 48.8 48.55) (end 49.125001 48.224999) (width 0.5) (layer F.Cu) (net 10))
 (segment (start 49.14999 50.44999) (end 48.8 50.1) (width 0.5) (layer F.Cu) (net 10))
 (segment (start 48.8 50.1) (end 48.8 48.55) (width 0.5) (layer F.Cu) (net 10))
 (segment (start 58.45001 50.44999) (end 49.14999 50.44999) (width 0.5) (layer F.Cu) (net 10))
 (segment (start 49.125001 46.724999) (end 49.2 46.65) (width 0.5) (layer F.Cu) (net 10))
 (segment (start 58.71 50.19) (end 58.45001 50.44999) (width 0.5) (layer F.Cu) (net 10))
 (segment (start 58.71 49.04) (end 58.71 50.19) (width 0.5) (layer F.Cu) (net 10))
 (segment (start 43.97 33.57) (end 43.97 31.5) (width 0.5) (layer F.Cu) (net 15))
 (segment (start 49.6 34) (end 44.4 34) (width 0.5) (layer F.Cu) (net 15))
 (segment (start 44.4 34) (end 43.97 33.57) (width 0.5) (layer F.Cu) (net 15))
 (segment (start 50 34.4) (end 49.6 34) (width 0.5) (layer F.Cu) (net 15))
 (segment (start 50 38.15) (end 50 34.4) (width 0.5) (layer F.Cu) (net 15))
 (segment (start 44.4 35.5) (end 44.4 38.15) (width 0.5) (layer F.Cu) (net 14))
 (segment (start 43.9 35) (end 44.4 35.5) (width 0.5) (layer F.Cu) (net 14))
 (segment (start 41.8 35) (end 43.9 35) (width 0.5) (layer F.Cu) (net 14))
 (segment (start 41.43 34.63) (end 41.8 35) (width 0.5) (layer F.Cu) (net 14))
 (segment (start 41.43 31.5) (end 41.43 34.63) (width 0.5) (layer F.Cu) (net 14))
 (segment (start 39.2 36) (end 42.6 36) (width 0.5) (layer F.Cu) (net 13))
 (segment (start 38.89 35.69) (end 39.2 36) (width 0.5) (layer F.Cu) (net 13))
 (segment (start 42.95 36.35) (end 42.95 39.6) (width 0.5) (layer F.Cu) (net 13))
 (segment (start 42.6 36) (end 42.95 36.35) (width 0.5) (layer F.Cu) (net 13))
 (segment (start 38.89 31.5) (end 38.89 35.69) (width 0.5) (layer F.Cu) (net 13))
 (segment (start 69.6875 37.6) (end 69.6875 40.1) (width 0.5) (layer F.Cu) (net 18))
 (segment (start 69.6875 40.1) (end 69.6875 41.5625) (width 0.5) (layer F.Cu) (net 18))
 (segment (start 69.6875 41.5625) (end 69.05 42.2) (width 0.5) (layer F.Cu) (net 18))
 (segment (start 66.7875 44.2) (end 65 42.4125) (width 0.5) (layer F.Cu) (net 19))
 (segment (start 68.1 44.2) (end 66.7875 44.2) (width 0.5) (layer F.Cu) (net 19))
 (segment (start 51.45 40.4) (end 64.25 40.4) (width 0.5) (layer F.Cu) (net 20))
 (segment (start 64.25 40.4) (end 64.75 39.9) (width 0.5) (layer F.Cu) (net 20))
 (segment (start 64.75 39.9) (end 64.75 38.1) (width 0.5) (layer F.Cu) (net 20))
 (segment (start 65.25 37.6) (end 66.7125 37.6) (width 0.5) (layer F.Cu) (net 20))
 (segment (start 64.75 38.1) (end 65.25 37.6) (width 0.5) (layer F.Cu) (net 20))
 (segment (start 51.8 38.1) (end 54.5125 38.1) (width 0.5) (layer F.Cu) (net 21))
 (segment (start 51.45 38.45) (end 51.8 38.1) (width 0.5) (layer F.Cu) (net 21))
 (segment (start 51.45 39.6) (end 51.45 38.45) (width 0.5) (layer F.Cu) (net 21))
 (segment (start 41.65 40.4) (end 42.95 40.4) (width 0.5) (layer F.Cu) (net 12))
 (segment (start 41.2 39.95) (end 41.65 40.4) (width 0.5) (layer F.Cu) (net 12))
 (segment (start 40.7 37) (end 41.2 37.5) (width 0.5) (layer F.Cu) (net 12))
 (segment (start 36.7 37) (end 40.7 37) (width 0.5) (layer F.Cu) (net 12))
 (segment (start 41.2 37.5) (end 41.2 39.95) (width 0.5) (layer F.Cu) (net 12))
 (segment (start 36.35 36.65) (end 36.7 37) (width 0.5) (layer F.Cu) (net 12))
 (segment (start 36.35 31.5) (end 36.35 36.65) (width 0.5) (layer F.Cu) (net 12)))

